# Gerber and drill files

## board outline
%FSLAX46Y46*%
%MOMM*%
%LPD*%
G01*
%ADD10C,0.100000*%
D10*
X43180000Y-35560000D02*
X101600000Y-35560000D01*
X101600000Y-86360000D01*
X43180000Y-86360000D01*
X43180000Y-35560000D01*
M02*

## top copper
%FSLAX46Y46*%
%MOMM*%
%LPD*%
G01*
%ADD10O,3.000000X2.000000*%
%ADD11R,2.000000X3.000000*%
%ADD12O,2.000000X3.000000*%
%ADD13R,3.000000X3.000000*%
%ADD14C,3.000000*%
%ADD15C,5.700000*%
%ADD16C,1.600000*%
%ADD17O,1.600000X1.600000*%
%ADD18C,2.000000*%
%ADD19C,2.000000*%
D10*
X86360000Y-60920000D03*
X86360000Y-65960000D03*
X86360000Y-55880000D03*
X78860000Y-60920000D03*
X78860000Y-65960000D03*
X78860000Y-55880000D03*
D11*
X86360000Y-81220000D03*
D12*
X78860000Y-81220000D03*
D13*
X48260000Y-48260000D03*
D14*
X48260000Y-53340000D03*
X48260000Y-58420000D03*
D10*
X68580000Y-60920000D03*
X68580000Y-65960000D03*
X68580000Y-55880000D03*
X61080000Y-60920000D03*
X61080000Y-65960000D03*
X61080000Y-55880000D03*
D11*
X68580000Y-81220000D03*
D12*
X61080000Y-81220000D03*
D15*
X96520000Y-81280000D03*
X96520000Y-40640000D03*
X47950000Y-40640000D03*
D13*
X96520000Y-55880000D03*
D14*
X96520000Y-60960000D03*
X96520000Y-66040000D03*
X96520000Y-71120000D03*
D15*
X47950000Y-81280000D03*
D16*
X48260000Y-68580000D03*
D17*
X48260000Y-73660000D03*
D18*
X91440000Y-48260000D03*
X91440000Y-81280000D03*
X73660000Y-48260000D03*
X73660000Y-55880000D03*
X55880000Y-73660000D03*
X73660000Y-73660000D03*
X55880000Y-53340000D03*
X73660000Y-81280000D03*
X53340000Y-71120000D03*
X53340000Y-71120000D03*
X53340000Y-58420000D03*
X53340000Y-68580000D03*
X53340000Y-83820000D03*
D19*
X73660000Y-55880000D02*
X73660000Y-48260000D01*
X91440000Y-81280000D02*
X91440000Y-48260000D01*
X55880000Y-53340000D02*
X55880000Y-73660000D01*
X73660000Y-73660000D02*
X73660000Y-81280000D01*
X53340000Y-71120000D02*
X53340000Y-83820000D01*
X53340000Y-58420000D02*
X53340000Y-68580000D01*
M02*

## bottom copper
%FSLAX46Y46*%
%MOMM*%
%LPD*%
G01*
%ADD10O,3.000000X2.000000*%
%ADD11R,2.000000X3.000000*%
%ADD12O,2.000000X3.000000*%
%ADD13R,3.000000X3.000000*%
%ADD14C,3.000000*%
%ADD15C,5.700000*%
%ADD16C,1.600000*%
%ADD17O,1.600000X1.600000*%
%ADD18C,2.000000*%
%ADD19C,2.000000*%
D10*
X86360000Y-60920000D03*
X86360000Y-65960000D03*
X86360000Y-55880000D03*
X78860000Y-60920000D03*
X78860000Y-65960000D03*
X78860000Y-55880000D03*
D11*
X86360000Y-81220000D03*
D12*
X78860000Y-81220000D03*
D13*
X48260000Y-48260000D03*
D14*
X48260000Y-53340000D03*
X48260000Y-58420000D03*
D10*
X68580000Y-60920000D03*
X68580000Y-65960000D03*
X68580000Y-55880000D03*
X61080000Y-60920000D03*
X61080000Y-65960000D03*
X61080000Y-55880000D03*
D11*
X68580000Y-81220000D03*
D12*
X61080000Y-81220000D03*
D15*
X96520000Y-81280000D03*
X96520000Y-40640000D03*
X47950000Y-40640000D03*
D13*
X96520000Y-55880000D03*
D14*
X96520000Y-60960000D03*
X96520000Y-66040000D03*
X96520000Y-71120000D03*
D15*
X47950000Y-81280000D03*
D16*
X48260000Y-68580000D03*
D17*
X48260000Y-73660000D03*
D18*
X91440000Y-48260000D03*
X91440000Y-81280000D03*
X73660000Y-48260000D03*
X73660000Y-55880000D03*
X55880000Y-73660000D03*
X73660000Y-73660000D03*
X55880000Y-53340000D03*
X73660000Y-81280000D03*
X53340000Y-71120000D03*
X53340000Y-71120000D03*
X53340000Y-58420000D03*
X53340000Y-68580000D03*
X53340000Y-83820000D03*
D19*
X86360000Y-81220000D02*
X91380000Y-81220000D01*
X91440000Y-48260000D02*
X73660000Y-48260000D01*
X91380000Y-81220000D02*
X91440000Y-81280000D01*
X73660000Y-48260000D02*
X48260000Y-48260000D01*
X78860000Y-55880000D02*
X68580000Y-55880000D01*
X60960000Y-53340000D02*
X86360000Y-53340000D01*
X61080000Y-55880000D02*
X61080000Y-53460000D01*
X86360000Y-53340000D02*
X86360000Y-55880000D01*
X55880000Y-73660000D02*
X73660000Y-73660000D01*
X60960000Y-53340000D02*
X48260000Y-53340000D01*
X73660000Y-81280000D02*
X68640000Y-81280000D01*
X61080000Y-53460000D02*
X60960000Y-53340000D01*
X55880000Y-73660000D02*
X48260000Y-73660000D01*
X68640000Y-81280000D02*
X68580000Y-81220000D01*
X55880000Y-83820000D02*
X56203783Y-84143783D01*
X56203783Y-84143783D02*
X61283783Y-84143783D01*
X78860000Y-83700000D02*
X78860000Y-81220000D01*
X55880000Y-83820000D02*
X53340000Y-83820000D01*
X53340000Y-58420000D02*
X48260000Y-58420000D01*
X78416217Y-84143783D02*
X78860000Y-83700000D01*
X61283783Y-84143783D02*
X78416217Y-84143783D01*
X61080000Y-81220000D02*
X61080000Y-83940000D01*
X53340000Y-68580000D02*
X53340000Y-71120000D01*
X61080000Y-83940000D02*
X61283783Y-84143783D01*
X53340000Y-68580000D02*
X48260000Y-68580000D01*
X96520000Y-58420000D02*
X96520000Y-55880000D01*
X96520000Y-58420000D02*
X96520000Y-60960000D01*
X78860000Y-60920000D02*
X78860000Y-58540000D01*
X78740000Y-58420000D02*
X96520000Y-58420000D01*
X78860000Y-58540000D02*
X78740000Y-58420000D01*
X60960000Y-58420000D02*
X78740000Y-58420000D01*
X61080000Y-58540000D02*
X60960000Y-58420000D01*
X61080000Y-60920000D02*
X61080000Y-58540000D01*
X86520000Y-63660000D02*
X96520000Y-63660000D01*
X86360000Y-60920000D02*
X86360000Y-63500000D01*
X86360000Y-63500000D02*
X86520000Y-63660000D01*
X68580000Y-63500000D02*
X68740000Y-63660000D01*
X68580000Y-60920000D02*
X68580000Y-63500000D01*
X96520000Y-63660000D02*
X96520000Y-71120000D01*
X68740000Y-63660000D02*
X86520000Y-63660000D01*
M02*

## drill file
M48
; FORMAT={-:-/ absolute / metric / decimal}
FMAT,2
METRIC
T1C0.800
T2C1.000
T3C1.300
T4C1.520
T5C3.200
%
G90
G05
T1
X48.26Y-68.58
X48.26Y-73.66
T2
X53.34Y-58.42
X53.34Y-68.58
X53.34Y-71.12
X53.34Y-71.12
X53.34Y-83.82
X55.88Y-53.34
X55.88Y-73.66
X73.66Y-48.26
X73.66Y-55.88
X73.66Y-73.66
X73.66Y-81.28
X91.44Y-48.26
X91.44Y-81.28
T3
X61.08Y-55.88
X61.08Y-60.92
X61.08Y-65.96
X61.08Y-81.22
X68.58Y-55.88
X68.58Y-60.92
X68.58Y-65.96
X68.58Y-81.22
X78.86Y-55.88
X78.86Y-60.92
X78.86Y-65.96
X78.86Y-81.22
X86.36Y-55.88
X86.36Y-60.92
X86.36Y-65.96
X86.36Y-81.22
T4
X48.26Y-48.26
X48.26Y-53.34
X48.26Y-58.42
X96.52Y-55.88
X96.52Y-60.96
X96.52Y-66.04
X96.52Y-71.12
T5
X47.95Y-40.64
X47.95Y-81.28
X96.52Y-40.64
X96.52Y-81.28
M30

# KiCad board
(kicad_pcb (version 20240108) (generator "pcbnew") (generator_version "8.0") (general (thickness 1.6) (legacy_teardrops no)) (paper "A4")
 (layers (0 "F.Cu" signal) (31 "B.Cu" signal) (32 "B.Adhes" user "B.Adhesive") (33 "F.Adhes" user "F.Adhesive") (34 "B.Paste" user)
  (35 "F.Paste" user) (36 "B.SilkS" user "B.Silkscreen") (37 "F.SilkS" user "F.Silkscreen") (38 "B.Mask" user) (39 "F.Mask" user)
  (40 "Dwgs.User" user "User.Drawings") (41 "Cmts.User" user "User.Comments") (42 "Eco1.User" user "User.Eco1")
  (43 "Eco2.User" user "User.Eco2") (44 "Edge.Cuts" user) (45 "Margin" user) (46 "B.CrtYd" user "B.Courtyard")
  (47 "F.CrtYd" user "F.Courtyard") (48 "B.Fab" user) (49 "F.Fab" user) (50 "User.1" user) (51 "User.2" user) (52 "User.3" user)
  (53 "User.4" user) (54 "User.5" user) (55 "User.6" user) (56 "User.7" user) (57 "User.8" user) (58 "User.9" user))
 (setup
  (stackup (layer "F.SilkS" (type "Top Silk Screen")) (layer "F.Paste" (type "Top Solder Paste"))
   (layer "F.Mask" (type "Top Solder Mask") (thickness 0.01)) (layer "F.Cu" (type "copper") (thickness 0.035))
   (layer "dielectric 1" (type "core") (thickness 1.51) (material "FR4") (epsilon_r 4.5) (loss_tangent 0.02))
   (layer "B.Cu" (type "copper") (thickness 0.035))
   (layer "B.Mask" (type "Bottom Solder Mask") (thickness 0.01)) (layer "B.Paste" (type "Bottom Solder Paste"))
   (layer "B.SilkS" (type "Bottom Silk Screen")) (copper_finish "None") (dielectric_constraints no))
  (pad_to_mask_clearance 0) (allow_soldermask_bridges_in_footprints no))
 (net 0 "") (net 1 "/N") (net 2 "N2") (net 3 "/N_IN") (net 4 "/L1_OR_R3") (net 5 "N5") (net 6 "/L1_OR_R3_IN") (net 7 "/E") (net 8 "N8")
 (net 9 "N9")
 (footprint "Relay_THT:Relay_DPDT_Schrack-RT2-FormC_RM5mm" (layer "F.Cu") (at 86.36 81.22 90)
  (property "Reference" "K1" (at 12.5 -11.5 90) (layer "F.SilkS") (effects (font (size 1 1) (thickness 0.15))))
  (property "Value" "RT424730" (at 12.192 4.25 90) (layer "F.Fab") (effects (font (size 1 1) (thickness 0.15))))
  (pad "11" thru_hole oval (at 20.3 0 270) (size 2 3) (drill 1.3) (layers "*.Cu" "*.Mask") (remove_unused_layers no) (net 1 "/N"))
  (pad "12" thru_hole oval (at 15.26 0 270) (size 2 3) (drill 1.3) (layers "*.Cu" "*.Mask") (remove_unused_layers no) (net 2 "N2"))
  (pad "14" thru_hole oval (at 25.34 0 270) (size 2 3) (drill 1.3) (layers "*.Cu" "*.Mask") (remove_unused_layers no) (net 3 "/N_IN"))
  (pad "21" thru_hole oval (at 20.3 -7.5 270) (size 2 3) (drill 1.3) (layers "*.Cu" "*.Mask") (remove_unused_layers no) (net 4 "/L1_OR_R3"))
  (pad "22" thru_hole oval (at 15.26 -7.5 270) (size 2 3) (drill 1.3) (layers "*.Cu" "*.Mask") (remove_unused_layers no) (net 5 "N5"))
  (pad "24" thru_hole oval (at 25.34 -7.5 270) (size 2 3) (drill 1.3) (layers "*.Cu" "*.Mask") (remove_unused_layers no)
   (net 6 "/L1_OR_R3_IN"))
  (pad "A1" thru_hole rect (at 0 0 270) (size 3 2) (drill 1.3) (layers "*.Cu" "*.Mask") (remove_unused_layers no) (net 6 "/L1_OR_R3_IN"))
  (pad "A2" thru_hole oval (at 0 -7.5 270) (size 3 2) (drill 1.3) (layers "*.Cu" "*.Mask") (remove_unused_layers no) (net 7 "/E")))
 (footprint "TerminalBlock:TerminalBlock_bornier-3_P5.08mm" (layer "F.Cu") (at 48.26 48.26 -90)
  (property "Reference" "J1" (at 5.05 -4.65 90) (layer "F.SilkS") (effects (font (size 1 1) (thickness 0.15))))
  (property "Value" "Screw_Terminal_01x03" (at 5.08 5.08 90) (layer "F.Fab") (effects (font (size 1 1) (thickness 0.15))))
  (pad "1" thru_hole rect (at 0 0 270) (size 3 3) (drill 1.52) (layers "*.Cu" "*.Mask") (remove_unused_layers no) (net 6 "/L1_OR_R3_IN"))
  (pad "2" thru_hole circle (at 5.08 0 270) (size 3 3) (drill 1.52) (layers "*.Cu" "*.Mask") (remove_unused_layers no) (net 3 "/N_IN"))
  (pad "3" thru_hole circle (at 10.16 0 270) (size 3 3) (drill 1.52) (layers "*.Cu" "*.Mask") (remove_unused_layers no) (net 7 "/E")))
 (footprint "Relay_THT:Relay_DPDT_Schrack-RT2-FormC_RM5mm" (layer "F.Cu") (at 68.58 81.22 90)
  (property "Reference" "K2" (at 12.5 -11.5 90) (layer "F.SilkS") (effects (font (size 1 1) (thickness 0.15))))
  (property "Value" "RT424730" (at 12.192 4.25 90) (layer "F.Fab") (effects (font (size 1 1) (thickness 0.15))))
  (pad "11" thru_hole oval (at 20.3 0 270) (size 2 3) (drill 1.3) (layers "*.Cu" "*.Mask") (remove_unused_layers no) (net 1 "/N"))
  (pad "12" thru_hole oval (at 15.26 0 270) (size 2 3) (drill 1.3) (layers "*.Cu" "*.Mask") (remove_unused_layers no) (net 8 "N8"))
  (pad "14" thru_hole oval (at 25.34 0 270) (size 2 3) (drill 1.3) (layers "*.Cu" "*.Mask") (remove_unused_layers no) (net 6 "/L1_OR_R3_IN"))
  (pad "21" thru_hole oval (at 20.3 -7.5 270) (size 2 3) (drill 1.3) (layers "*.Cu" "*.Mask") (remove_unused_layers no) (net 4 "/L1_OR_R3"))
  (pad "22" thru_hole oval (at 15.26 -7.5 270) (size 2 3) (drill 1.3) (layers "*.Cu" "*.Mask") (remove_unused_layers no) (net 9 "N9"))
  (pad "24" thru_hole oval (at 25.34 -7.5 270) (size 2 3) (drill 1.3) (layers "*.Cu" "*.Mask") (remove_unused_layers no) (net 3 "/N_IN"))
  (pad "A1" thru_hole rect (at 0 0 270) (size 3 2) (drill 1.3) (layers "*.Cu" "*.Mask") (remove_unused_layers no) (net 3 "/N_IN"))
  (pad "A2" thru_hole oval (at 0 -7.5 270) (size 3 2) (drill 1.3) (layers "*.Cu" "*.Mask") (remove_unused_layers no) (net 7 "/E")))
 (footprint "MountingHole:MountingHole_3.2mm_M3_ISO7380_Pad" (layer "F.Cu") (at 96.52 81.28)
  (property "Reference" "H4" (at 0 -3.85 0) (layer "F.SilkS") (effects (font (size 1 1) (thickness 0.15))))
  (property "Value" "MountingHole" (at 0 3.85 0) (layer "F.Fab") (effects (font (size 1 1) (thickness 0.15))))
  (pad "1" thru_hole circle (at 0 0) (size 5.7 5.7) (drill 3.2) (layers "*.Cu" "*.Mask") (remove_unused_layers no)))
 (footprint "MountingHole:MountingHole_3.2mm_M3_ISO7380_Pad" (layer "F.Cu") (at 96.52 40.64)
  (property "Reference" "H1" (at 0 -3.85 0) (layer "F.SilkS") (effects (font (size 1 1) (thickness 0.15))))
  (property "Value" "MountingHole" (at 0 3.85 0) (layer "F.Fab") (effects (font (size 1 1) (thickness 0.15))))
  (pad "1" thru_hole circle (at 0 0) (size 5.7 5.7) (drill 3.2) (layers "*.Cu" "*.Mask") (remove_unused_layers no)))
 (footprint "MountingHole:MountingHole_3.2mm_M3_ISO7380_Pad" (layer "F.Cu") (at 47.95 40.64)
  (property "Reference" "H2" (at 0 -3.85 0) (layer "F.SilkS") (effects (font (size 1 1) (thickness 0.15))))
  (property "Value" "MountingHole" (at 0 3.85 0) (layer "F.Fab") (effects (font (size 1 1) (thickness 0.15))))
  (pad "1" thru_hole circle (at 0 0) (size 5.7 5.7) (drill 3.2) (layers "*.Cu" "*.Mask") (remove_unused_layers no)))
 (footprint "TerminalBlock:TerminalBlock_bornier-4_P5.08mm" (layer "F.Cu") (at 96.52 55.88 -90)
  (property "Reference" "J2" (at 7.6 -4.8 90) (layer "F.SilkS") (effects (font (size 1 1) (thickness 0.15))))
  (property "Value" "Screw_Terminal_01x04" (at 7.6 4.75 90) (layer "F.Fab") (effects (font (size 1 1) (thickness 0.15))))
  (pad "1" thru_hole rect (at 0 0 270) (size 3 3) (drill 1.52) (layers "*.Cu" "*.Mask") (remove_unused_layers no) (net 4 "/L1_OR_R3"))
  (pad "2" thru_hole circle (at 5.08 0 270) (size 3 3) (drill 1.52) (layers "*.Cu" "*.Mask") (remove_unused_layers no) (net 4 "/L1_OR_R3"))
  (pad "3" thru_hole circle (at 10.16 0 270) (size 3 3) (drill 1.52) (layers "*.Cu" "*.Mask") (remove_unused_layers no) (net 1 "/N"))
  (pad "4" thru_hole circle (at 15.24 0 270) (size 3 3) (drill 1.52) (layers "*.Cu" "*.Mask") (remove_unused_layers no) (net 1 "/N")))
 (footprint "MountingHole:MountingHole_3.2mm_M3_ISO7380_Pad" (layer "F.Cu") (at 47.95 81.28)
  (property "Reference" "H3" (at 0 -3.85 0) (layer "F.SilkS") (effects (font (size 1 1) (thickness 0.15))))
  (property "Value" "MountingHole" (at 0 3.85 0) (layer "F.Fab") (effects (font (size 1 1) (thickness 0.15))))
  (pad "1" thru_hole circle (at 0 0) (size 5.7 5.7) (drill 3.2) (layers "*.Cu" "*.Mask") (remove_unused_layers no)))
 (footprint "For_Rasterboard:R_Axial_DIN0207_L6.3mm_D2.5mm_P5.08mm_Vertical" (layer "F.Cu") (at 48.26 68.58 -90)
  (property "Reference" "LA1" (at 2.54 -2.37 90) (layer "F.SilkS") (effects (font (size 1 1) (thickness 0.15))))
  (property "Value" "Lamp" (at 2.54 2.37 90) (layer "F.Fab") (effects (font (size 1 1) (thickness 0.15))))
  (pad "1" thru_hole circle (at 0 0 270) (size 1.6 1.6) (drill 0.8) (layers "*.Cu" "*.Mask") (remove_unused_layers no) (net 7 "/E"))
  (pad "2" thru_hole oval (at 5.08 0 270) (size 1.6 1.6) (drill 0.8) (layers "*.Cu" "*.Mask") (remove_unused_layers no) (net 3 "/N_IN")))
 (gr_rect (start 43.18 35.56) (end 101.6 86.36) (stroke (width 0.1) (type solid)) (fill none) (layer "Edge.Cuts"))
 (segment (start 73.66 55.88) (end 73.66 48.26) (width 2) (layer "F.Cu") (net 6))
 (segment (start 91.44 81.28) (end 91.44 48.26) (width 2) (layer "F.Cu") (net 6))
 (via (at 91.44 48.26) (size 2) (drill 1) (layers "F.Cu" "B.Cu") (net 6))
 (via (at 91.44 81.28) (size 2) (drill 1) (layers "F.Cu" "B.Cu") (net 6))
 (via (at 73.66 48.26) (size 2) (drill 1) (layers "F.Cu" "B.Cu") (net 6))
 (via (at 73.66 55.88) (size 2) (drill 1) (layers "F.Cu" "B.Cu") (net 6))
 (segment (start 86.36 81.22) (end 91.38 81.22) (width 2) (layer "B.Cu") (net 6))
 (segment (start 91.44 48.26) (end 73.66 48.26) (width 2) (layer "B.Cu") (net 6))
 (segment (start 91.38 81.22) (end 91.44 81.28) (width 2) (layer "B.Cu") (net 6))
 (segment (start 73.66 48.26) (end 48.26 48.26) (width 2) (layer "B.Cu") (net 6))
 (segment (start 78.86 55.88) (end 68.58 55.88) (width 2) (layer "B.Cu") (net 6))
 (segment (start 55.88 53.34) (end 55.88 73.66) (width 2) (layer "F.Cu") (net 3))
 (segment (start 73.66 73.66) (end 73.66 81.28) (width 2) (layer "F.Cu") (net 3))
 (via (at 55.88 73.66) (size 2) (drill 1) (layers "F.Cu" "B.Cu") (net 3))
 (via (at 73.66 73.66) (size 2) (drill 1) (layers "F.Cu" "B.Cu") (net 3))
 (via (at 55.88 53.34) (size 2) (drill 1) (layers "F.Cu" "B.Cu") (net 3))
 (via (at 73.66 81.28) (size 2) (drill 1) (layers "F.Cu" "B.Cu") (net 3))
 (segment (start 60.96 53.34) (end 86.36 53.34) (width 2) (layer "B.Cu") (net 3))
 (segment (start 61.08 55.88) (end 61.08 53.46) (width 2) (layer "B.Cu") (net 3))
 (segment (start 86.36 53.34) (end 86.36 55.88) (width 2) (layer "B.Cu") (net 3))
 (segment (start 55.88 73.66) (end 73.66 73.66) (width 2) (layer "B.Cu") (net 3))
 (segment (start 60.96 53.34) (end 48.26 53.34) (width 2) (layer "B.Cu") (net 3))
 (segment (start 73.66 81.28) (end 68.64 81.28) (width 2) (layer "B.Cu") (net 3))
 (segment (start 61.08 53.46) (end 60.96 53.34) (width 2) (layer "B.Cu") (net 3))
 (segment (start 55.88 73.66) (end 48.26 73.66) (width 2) (layer "B.Cu") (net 3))
 (segment (start 68.64 81.28) (end 68.58 81.22) (width 2) (layer "B.Cu") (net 3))
 (segment (start 53.34 71.12) (end 53.34 83.82) (width 2) (layer "F.Cu") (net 7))
 (segment (start 53.34 58.42) (end 53.34 68.58) (width 2) (layer "F.Cu") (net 7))
 (via (at 53.34 71.12) (size 2) (drill 1) (layers "F.Cu" "B.Cu") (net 7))
 (via (at 53.34 71.12) (size 2) (drill 1) (layers "F.Cu" "B.Cu") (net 7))
 (via (at 53.34 58.42) (size 2) (drill 1) (layers "F.Cu" "B.Cu") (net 7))
 (via (at 53.34 68.58) (size 2) (drill 1) (layers "F.Cu" "B.Cu") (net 7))
 (via (at 53.34 83.82) (size 2) (drill 1) (layers "F.Cu" "B.Cu") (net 7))
 (segment (start 55.88 83.82) (end 56.203783 84.143783) (width 2) (layer "B.Cu") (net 7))
 (segment (start 56.203783 84.143783) (end 61.283783 84.143783) (width 2) (layer "B.Cu") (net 7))
 (segment (start 78.86 83.7) (end 78.86 81.22) (width 2) (layer "B.Cu") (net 7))
 (segment (start 55.88 83.82) (end 53.34 83.82) (width 2) (layer "B.Cu") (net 7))
 (segment (start 53.34 58.42) (end 48.26 58.42) (width 2) (layer "B.Cu") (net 7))
 (segment (start 78.416217 84.143783) (end 78.86 83.7) (width 2) (layer "B.Cu") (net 7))
 (segment (start 61.283783 84.143783) (end 78.416217 84.143783) (width 2) (layer "B.Cu") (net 7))
 (segment (start 61.08 81.22) (end 61.08 83.94) (width 2) (layer "B.Cu") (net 7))
 (segment (start 53.34 68.58) (end 53.34 71.12) (width 2) (layer "B.Cu") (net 7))
 (segment (start 61.08 83.94) (end 61.283783 84.143783) (width 2) (layer "B.Cu") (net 7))
 (segment (start 53.34 68.58) (end 48.26 68.58) (width 2) (layer "B.Cu") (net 7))
 (segment (start 96.52 58.42) (end 96.52 55.88) (width 2) (layer "B.Cu") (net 4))
 (segment (start 96.52 58.42) (end 96.52 60.96) (width 2) (layer "B.Cu") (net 4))
 (segment (start 78.86 60.92) (end 78.86 58.54) (width 2) (layer "B.Cu") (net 4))
 (segment (start 78.74 58.42) (end 96.52 58.42) (width 2) (layer "B.Cu") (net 4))
 (segment (start 78.86 58.54) (end 78.74 58.42) (width 2) (layer "B.Cu") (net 4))
 (segment (start 60.96 58.42) (end 78.74 58.42) (width 2) (layer "B.Cu") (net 4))
 (segment (start 61.08 58.54) (end 60.96 58.42) (width 2) (layer "B.Cu") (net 4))
 (segment (start 61.08 60.92) (end 61.08 58.54) (width 2) (layer "B.Cu") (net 4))
 (segment (start 86.52 63.66) (end 96.52 63.66) (width 2) (layer "B.Cu") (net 1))
 (segment (start 86.36 60.92) (end 86.36 63.5) (width 2) (layer "B.Cu") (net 1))
 (segment (start 86.36 63.5) (end 86.52 63.66) (width 2) (layer "B.Cu") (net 1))
 (segment (start 68.58 63.5) (end 68.74 63.66) (width 2) (layer "B.Cu") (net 1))
 (segment (start 68.58 60.92) (end 68.58 63.5) (width 2) (layer "B.Cu") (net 1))
 (segment (start 96.52 63.66) (end 96.52 71.12) (width 2) (layer "B.Cu") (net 1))
 (segment (start 68.74 63.66) (end 86.52 63.66) (width 2) (layer "B.Cu") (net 1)))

